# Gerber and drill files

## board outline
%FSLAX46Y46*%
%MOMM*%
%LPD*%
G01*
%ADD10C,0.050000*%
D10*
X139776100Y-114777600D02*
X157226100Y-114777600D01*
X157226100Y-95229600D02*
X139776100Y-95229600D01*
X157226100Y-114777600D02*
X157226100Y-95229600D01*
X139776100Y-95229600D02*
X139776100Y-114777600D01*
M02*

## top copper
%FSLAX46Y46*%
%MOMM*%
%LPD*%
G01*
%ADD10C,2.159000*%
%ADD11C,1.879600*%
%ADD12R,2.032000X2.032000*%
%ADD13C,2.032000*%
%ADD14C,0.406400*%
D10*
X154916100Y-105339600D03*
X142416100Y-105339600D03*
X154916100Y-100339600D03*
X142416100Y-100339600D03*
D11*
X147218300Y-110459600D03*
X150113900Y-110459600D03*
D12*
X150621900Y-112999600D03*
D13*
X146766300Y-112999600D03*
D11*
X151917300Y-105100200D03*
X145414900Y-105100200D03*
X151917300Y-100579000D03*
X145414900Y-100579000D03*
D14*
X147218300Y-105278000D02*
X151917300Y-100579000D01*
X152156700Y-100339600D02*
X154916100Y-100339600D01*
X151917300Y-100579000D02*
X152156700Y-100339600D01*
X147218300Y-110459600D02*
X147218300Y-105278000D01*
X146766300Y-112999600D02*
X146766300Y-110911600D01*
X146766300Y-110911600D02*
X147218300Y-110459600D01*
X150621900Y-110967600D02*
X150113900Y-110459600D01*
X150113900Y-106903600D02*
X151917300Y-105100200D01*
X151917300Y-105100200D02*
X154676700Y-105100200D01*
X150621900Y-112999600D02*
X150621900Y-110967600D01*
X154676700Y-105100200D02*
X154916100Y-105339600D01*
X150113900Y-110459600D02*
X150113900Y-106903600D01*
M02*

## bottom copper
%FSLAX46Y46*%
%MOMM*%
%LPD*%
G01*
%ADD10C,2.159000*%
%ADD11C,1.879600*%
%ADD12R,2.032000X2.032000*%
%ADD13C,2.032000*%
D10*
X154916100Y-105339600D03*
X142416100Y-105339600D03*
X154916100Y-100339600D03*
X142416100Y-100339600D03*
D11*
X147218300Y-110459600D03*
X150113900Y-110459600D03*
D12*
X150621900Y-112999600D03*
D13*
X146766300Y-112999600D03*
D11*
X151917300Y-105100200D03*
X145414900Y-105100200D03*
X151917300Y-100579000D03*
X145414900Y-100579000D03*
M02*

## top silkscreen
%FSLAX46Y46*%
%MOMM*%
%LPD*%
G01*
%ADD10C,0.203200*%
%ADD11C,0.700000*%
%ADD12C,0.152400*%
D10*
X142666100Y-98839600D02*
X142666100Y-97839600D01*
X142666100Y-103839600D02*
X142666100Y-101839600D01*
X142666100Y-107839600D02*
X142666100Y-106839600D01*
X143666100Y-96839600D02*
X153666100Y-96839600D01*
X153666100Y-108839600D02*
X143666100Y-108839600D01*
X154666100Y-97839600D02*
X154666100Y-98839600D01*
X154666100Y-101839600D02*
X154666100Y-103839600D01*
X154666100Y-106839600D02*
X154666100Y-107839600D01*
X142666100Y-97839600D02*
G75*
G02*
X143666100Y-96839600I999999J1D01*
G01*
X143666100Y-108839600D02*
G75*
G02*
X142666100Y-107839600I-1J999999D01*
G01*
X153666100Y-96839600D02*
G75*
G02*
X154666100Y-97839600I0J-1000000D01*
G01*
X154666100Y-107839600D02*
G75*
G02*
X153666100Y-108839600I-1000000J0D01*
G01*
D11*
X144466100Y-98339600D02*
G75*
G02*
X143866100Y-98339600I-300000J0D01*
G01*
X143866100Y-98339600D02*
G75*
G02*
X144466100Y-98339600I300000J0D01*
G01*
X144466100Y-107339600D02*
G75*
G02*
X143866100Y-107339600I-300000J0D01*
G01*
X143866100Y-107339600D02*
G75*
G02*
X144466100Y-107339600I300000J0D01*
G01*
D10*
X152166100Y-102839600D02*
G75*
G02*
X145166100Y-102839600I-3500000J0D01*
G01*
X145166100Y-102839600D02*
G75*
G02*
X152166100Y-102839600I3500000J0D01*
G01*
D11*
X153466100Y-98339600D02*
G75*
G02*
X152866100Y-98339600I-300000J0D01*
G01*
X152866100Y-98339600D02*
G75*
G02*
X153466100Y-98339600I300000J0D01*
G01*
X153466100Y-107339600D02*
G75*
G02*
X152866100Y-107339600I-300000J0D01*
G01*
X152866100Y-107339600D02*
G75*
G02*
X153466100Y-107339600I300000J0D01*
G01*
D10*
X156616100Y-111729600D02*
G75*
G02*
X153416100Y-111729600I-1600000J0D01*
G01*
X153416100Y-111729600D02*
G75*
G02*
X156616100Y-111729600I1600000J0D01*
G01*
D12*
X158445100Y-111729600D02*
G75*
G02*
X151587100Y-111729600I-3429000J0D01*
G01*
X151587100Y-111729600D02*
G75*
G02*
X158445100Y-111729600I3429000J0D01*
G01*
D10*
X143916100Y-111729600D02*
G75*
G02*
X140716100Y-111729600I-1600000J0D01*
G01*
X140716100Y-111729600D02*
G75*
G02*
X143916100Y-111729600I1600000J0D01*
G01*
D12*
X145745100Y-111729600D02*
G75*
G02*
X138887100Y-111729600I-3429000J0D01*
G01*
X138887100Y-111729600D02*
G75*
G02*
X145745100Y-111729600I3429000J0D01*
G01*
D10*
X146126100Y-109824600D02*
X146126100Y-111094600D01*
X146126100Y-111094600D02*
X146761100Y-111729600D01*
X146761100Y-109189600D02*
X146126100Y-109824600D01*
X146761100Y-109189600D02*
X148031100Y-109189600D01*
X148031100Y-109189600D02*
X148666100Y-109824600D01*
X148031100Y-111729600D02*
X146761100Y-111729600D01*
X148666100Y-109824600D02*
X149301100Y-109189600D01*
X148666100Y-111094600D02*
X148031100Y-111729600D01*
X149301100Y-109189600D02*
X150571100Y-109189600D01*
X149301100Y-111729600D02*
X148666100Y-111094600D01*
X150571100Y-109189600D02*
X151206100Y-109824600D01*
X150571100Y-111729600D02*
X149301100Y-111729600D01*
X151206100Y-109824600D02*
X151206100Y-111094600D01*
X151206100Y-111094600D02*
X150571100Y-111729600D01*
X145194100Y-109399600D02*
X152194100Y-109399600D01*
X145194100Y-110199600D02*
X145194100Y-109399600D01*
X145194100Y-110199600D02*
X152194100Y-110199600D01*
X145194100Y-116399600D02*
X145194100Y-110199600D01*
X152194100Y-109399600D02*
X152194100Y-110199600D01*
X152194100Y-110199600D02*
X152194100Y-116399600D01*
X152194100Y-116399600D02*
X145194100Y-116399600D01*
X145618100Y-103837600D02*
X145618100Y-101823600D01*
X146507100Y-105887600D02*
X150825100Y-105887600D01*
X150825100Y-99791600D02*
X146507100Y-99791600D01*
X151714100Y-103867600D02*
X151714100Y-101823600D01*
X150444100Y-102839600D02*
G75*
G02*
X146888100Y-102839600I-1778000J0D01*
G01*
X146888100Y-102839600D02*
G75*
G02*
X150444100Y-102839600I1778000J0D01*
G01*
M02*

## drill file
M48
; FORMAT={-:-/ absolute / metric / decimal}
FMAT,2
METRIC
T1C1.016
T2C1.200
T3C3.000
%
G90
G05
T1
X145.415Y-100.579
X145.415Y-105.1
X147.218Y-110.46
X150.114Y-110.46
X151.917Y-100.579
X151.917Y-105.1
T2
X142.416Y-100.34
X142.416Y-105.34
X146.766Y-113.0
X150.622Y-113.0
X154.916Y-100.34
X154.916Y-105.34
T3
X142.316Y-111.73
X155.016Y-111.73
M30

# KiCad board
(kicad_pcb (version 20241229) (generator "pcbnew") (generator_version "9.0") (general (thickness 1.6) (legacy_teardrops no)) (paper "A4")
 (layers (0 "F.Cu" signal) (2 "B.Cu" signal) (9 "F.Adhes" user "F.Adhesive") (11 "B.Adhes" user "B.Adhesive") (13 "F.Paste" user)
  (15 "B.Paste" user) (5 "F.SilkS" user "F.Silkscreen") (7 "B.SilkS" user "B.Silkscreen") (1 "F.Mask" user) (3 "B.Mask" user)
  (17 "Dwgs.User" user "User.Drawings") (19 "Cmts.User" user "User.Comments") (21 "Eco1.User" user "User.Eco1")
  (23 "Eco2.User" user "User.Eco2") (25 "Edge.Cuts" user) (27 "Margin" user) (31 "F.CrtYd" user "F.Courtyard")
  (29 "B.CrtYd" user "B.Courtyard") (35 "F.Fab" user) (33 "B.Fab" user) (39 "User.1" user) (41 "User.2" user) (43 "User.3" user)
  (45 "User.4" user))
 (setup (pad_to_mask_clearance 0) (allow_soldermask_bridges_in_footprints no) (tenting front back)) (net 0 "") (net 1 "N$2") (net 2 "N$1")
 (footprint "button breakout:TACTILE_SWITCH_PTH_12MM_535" (layer "F.Cu") (at 148.6661 102.8396)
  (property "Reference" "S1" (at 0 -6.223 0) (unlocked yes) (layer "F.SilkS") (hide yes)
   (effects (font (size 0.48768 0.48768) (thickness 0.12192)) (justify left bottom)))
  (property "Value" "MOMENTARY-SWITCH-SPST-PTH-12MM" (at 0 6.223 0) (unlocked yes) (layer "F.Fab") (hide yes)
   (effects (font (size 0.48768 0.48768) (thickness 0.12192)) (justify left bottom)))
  (fp_line (start -6 -4) (end -6 -5) (stroke (width 0.2032) (type solid)) (layer "F.SilkS"))
  (fp_line (start -6 1) (end -6 -1) (stroke (width 0.2032) (type solid)) (layer "F.SilkS"))
  (fp_line (start -6 5) (end -6 4) (stroke (width 0.2032) (type solid)) (layer "F.SilkS"))
  (fp_line (start -5 -6) (end 5 -6) (stroke (width 0.2032) (type solid)) (layer "F.SilkS"))
  (fp_line (start 5 6) (end -5 6) (stroke (width 0.2032) (type solid)) (layer "F.SilkS"))
  (fp_line (start 6 -5) (end 6 -4) (stroke (width 0.2032) (type solid)) (layer "F.SilkS"))
  (fp_line (start 6 -1) (end 6 1) (stroke (width 0.2032) (type solid)) (layer "F.SilkS"))
  (fp_line (start 6 4) (end 6 5) (stroke (width 0.2032) (type solid)) (layer "F.SilkS"))
  (fp_arc (start -6 -5) (mid -5.707107 -5.707107) (end -5 -6) (stroke (width 0.2032) (type solid)) (layer "F.SilkS"))
  (fp_arc (start -5 6) (mid -5.707107 5.707107) (end -6 5) (stroke (width 0.2032) (type solid)) (layer "F.SilkS"))
  (fp_arc (start 5 -6) (mid 5.707107 -5.707107) (end 6 -5) (stroke (width 0.2032) (type solid)) (layer "F.SilkS"))
  (fp_arc (start 6 5) (mid 5.707107 5.707107) (end 5 6) (stroke (width 0.2032) (type solid)) (layer "F.SilkS"))
  (fp_circle (center -4.5 -4.5) (end -4.2 -4.5) (stroke (width 0.7) (type solid)) (fill no) (layer "F.SilkS"))
  (fp_circle (center -4.5 4.5) (end -4.2 4.5) (stroke (width 0.7) (type solid)) (fill no) (layer "F.SilkS"))
  (fp_circle (center 0 0) (end 3.5 0) (stroke (width 0.2032) (type solid)) (fill no) (layer "F.SilkS"))
  (fp_circle (center 4.5 -4.5) (end 4.8 -4.5) (stroke (width 0.7) (type solid)) (fill no) (layer "F.SilkS"))
  (fp_circle (center 4.5 4.5) (end 4.8 4.5) (stroke (width 0.7) (type solid)) (fill no) (layer "F.SilkS"))
  (pad "1" thru_hole circle (at 6.25 2.5) (size 2.159 2.159) (drill 1.2) (layers "*.Cu" "*.Mask") (remove_unused_layers no) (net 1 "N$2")
   (solder_mask_margin 0.0508) (thermal_bridge_angle 0))
  (pad "2" thru_hole circle (at -6.25 2.5) (size 2.159 2.159) (drill 1.2) (layers "*.Cu" "*.Mask") (remove_unused_layers no)
   (solder_mask_margin 0.0508) (thermal_bridge_angle 0))
  (pad "3" thru_hole circle (at 6.25 -2.5) (size 2.159 2.159) (drill 1.2) (layers "*.Cu" "*.Mask") (remove_unused_layers no) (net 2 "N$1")
   (solder_mask_margin 0.0508) (thermal_bridge_angle 0))
  (pad "4" thru_hole circle (at -6.25 -2.5) (size 2.159 2.159) (drill 1.2) (layers "*.Cu" "*.Mask") (remove_unused_layers no)
   (solder_mask_margin 0.0508) (thermal_bridge_angle 0)))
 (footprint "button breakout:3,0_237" (layer "F.Cu") (at 155.0161 111.7296)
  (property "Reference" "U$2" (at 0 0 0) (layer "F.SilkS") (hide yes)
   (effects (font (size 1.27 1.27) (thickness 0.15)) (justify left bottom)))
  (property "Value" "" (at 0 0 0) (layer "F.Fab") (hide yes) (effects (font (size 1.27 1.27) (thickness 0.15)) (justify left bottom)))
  (fp_circle (center 0 0) (end 1.6 0) (stroke (width 0.2032) (type solid)) (fill no) (layer "F.SilkS"))
  (fp_circle (center 0 0) (end 3.429 0) (stroke (width 0.1524) (type solid)) (fill no) (layer "F.SilkS"))
  (pad "" np_thru_hole circle (at 0 0) (size 3 3) (drill 3) (layers "*.Cu" "*.Mask"))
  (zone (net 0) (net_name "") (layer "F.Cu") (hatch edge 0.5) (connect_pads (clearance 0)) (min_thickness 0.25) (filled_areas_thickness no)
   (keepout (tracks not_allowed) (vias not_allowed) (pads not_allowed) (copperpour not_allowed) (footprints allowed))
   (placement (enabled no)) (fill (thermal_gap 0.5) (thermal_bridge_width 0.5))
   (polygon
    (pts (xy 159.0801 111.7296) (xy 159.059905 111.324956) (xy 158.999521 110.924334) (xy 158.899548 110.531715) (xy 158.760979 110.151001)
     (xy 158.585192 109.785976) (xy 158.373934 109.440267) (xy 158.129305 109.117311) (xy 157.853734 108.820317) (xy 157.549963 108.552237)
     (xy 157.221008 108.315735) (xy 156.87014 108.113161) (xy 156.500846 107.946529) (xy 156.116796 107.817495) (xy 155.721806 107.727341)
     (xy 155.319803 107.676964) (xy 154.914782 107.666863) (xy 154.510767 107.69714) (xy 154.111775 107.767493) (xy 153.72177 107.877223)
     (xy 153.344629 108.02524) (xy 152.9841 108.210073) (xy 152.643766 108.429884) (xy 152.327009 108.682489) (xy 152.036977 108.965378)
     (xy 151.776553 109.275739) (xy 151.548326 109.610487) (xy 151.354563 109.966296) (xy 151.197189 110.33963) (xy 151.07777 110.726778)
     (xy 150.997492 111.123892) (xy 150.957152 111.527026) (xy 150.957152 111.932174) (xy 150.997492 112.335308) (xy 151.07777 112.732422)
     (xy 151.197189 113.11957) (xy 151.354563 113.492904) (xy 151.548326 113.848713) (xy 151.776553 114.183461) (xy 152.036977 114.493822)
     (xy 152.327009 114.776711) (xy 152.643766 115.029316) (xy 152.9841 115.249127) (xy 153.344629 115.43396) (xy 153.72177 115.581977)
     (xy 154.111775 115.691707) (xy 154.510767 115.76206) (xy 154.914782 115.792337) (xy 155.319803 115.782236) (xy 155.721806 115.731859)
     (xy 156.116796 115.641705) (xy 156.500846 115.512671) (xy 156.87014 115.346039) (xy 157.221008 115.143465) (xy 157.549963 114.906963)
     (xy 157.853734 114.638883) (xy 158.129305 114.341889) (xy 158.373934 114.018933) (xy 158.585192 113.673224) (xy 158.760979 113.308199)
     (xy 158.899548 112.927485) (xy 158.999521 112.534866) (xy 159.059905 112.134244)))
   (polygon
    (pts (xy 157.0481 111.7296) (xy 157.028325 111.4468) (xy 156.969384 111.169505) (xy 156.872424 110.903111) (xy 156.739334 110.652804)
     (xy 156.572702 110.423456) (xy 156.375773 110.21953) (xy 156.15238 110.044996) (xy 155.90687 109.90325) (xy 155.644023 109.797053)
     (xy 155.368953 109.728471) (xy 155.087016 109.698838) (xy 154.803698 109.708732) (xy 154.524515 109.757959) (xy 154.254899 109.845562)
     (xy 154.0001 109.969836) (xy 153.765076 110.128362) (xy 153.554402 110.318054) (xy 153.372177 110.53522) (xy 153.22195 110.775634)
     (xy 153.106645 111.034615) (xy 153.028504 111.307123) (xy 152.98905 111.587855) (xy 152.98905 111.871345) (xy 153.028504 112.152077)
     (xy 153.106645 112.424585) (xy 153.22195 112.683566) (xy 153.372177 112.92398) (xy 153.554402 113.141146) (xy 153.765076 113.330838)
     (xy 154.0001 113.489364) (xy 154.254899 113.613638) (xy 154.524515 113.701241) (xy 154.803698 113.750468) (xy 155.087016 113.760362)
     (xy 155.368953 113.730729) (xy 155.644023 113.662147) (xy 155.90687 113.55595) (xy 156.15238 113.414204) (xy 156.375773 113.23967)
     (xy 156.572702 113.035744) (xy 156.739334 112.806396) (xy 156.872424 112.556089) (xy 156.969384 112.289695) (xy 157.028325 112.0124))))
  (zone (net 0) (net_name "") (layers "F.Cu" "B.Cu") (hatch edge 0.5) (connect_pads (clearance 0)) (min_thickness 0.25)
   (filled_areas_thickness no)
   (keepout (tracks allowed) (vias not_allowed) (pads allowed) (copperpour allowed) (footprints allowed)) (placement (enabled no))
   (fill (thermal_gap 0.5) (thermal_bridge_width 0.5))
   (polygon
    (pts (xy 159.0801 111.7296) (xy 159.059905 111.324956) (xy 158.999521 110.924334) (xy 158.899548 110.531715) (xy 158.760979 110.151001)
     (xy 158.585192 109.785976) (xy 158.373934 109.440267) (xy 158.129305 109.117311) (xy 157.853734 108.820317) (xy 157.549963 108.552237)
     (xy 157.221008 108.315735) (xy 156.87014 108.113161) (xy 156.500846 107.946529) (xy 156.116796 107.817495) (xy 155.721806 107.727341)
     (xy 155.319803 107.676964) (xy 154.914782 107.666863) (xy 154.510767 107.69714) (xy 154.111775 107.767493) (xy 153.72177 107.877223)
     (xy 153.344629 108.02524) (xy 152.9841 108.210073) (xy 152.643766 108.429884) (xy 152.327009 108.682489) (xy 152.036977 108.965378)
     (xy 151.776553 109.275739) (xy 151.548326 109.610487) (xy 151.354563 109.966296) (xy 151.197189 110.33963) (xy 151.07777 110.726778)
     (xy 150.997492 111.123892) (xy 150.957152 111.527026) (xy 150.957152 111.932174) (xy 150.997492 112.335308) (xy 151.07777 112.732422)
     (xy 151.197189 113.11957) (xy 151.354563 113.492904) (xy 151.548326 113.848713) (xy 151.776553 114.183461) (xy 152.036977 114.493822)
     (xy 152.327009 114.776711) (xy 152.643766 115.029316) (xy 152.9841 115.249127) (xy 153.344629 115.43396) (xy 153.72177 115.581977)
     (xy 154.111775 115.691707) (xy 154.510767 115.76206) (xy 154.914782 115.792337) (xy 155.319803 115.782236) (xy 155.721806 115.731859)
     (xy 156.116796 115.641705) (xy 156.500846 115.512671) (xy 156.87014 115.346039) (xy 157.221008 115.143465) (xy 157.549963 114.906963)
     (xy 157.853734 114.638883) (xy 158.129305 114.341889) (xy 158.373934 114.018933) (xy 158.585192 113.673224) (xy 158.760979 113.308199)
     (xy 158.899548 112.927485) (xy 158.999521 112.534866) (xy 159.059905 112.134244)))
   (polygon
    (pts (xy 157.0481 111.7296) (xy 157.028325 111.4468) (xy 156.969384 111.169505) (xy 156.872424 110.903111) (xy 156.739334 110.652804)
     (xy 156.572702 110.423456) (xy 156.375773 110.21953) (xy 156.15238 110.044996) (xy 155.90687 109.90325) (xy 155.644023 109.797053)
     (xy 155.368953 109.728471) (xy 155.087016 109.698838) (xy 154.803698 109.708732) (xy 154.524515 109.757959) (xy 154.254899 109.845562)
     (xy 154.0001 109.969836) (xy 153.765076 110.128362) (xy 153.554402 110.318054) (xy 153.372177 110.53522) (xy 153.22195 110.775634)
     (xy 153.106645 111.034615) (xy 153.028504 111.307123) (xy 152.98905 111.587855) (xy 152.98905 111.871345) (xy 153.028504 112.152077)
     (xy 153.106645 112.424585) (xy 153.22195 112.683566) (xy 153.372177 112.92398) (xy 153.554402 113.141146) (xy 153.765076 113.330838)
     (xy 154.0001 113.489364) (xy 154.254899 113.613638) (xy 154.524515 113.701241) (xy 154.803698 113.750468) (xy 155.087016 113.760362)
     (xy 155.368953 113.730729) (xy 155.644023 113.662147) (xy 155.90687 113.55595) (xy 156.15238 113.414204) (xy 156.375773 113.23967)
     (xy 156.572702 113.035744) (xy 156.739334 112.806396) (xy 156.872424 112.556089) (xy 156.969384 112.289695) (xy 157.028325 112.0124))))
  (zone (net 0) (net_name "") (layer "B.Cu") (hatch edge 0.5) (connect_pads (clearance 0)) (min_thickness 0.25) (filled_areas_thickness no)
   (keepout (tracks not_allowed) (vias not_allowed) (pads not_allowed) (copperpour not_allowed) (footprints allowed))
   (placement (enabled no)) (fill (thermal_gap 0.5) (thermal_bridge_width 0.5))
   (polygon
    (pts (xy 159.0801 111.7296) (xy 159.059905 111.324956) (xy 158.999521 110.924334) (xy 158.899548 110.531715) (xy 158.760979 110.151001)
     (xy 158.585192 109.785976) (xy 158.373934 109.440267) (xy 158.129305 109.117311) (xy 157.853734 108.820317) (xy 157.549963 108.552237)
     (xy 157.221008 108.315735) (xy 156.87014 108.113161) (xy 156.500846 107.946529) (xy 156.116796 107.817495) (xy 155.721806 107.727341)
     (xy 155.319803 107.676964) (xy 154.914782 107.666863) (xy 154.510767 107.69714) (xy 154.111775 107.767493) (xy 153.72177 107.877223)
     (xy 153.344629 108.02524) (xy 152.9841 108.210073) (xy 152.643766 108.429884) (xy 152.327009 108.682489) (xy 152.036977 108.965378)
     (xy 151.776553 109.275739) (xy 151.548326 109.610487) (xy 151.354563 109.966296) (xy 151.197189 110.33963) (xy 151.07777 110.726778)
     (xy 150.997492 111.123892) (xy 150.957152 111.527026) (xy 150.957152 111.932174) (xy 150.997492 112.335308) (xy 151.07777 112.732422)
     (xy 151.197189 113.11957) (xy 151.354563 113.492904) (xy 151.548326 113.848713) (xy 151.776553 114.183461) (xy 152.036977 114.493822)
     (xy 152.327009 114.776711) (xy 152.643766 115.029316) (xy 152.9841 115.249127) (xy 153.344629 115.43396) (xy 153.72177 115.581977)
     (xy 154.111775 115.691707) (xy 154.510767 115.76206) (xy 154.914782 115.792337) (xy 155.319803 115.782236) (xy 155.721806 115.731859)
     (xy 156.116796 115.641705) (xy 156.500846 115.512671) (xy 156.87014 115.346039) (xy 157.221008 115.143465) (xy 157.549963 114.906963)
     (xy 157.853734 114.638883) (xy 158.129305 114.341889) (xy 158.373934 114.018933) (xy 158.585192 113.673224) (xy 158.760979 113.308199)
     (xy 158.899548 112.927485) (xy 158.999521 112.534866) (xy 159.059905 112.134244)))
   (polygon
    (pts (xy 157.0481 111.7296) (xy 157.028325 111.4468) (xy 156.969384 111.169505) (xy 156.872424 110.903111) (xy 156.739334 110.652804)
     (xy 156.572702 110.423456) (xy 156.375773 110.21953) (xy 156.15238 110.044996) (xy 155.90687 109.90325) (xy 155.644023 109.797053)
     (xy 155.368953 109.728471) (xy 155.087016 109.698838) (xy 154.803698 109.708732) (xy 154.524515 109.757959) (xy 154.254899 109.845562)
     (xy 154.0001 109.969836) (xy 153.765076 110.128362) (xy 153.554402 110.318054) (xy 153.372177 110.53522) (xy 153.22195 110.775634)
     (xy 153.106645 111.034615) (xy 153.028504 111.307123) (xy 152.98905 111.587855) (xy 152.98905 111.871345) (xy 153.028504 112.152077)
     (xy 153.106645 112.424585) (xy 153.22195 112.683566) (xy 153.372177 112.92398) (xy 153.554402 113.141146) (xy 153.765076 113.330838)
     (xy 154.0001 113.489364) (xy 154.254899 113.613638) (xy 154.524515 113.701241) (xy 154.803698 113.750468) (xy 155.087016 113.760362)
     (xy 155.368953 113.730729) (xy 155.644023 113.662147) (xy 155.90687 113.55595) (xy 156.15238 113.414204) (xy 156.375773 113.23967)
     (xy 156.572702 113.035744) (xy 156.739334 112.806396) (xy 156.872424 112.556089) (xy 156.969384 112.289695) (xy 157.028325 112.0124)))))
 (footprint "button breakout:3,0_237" (layer "F.Cu") (at 142.3161 111.7296)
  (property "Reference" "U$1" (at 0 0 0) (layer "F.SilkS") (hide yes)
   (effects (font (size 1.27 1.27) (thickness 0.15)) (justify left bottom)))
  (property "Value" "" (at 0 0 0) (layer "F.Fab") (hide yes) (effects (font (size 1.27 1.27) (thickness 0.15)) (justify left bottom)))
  (fp_circle (center 0 0) (end 1.6 0) (stroke (width 0.2032) (type solid)) (fill no) (layer "F.SilkS"))
  (fp_circle (center 0 0) (end 3.429 0) (stroke (width 0.1524) (type solid)) (fill no) (layer "F.SilkS"))
  (pad "" np_thru_hole circle (at 0 0) (size 3 3) (drill 3) (layers "*.Cu" "*.Mask"))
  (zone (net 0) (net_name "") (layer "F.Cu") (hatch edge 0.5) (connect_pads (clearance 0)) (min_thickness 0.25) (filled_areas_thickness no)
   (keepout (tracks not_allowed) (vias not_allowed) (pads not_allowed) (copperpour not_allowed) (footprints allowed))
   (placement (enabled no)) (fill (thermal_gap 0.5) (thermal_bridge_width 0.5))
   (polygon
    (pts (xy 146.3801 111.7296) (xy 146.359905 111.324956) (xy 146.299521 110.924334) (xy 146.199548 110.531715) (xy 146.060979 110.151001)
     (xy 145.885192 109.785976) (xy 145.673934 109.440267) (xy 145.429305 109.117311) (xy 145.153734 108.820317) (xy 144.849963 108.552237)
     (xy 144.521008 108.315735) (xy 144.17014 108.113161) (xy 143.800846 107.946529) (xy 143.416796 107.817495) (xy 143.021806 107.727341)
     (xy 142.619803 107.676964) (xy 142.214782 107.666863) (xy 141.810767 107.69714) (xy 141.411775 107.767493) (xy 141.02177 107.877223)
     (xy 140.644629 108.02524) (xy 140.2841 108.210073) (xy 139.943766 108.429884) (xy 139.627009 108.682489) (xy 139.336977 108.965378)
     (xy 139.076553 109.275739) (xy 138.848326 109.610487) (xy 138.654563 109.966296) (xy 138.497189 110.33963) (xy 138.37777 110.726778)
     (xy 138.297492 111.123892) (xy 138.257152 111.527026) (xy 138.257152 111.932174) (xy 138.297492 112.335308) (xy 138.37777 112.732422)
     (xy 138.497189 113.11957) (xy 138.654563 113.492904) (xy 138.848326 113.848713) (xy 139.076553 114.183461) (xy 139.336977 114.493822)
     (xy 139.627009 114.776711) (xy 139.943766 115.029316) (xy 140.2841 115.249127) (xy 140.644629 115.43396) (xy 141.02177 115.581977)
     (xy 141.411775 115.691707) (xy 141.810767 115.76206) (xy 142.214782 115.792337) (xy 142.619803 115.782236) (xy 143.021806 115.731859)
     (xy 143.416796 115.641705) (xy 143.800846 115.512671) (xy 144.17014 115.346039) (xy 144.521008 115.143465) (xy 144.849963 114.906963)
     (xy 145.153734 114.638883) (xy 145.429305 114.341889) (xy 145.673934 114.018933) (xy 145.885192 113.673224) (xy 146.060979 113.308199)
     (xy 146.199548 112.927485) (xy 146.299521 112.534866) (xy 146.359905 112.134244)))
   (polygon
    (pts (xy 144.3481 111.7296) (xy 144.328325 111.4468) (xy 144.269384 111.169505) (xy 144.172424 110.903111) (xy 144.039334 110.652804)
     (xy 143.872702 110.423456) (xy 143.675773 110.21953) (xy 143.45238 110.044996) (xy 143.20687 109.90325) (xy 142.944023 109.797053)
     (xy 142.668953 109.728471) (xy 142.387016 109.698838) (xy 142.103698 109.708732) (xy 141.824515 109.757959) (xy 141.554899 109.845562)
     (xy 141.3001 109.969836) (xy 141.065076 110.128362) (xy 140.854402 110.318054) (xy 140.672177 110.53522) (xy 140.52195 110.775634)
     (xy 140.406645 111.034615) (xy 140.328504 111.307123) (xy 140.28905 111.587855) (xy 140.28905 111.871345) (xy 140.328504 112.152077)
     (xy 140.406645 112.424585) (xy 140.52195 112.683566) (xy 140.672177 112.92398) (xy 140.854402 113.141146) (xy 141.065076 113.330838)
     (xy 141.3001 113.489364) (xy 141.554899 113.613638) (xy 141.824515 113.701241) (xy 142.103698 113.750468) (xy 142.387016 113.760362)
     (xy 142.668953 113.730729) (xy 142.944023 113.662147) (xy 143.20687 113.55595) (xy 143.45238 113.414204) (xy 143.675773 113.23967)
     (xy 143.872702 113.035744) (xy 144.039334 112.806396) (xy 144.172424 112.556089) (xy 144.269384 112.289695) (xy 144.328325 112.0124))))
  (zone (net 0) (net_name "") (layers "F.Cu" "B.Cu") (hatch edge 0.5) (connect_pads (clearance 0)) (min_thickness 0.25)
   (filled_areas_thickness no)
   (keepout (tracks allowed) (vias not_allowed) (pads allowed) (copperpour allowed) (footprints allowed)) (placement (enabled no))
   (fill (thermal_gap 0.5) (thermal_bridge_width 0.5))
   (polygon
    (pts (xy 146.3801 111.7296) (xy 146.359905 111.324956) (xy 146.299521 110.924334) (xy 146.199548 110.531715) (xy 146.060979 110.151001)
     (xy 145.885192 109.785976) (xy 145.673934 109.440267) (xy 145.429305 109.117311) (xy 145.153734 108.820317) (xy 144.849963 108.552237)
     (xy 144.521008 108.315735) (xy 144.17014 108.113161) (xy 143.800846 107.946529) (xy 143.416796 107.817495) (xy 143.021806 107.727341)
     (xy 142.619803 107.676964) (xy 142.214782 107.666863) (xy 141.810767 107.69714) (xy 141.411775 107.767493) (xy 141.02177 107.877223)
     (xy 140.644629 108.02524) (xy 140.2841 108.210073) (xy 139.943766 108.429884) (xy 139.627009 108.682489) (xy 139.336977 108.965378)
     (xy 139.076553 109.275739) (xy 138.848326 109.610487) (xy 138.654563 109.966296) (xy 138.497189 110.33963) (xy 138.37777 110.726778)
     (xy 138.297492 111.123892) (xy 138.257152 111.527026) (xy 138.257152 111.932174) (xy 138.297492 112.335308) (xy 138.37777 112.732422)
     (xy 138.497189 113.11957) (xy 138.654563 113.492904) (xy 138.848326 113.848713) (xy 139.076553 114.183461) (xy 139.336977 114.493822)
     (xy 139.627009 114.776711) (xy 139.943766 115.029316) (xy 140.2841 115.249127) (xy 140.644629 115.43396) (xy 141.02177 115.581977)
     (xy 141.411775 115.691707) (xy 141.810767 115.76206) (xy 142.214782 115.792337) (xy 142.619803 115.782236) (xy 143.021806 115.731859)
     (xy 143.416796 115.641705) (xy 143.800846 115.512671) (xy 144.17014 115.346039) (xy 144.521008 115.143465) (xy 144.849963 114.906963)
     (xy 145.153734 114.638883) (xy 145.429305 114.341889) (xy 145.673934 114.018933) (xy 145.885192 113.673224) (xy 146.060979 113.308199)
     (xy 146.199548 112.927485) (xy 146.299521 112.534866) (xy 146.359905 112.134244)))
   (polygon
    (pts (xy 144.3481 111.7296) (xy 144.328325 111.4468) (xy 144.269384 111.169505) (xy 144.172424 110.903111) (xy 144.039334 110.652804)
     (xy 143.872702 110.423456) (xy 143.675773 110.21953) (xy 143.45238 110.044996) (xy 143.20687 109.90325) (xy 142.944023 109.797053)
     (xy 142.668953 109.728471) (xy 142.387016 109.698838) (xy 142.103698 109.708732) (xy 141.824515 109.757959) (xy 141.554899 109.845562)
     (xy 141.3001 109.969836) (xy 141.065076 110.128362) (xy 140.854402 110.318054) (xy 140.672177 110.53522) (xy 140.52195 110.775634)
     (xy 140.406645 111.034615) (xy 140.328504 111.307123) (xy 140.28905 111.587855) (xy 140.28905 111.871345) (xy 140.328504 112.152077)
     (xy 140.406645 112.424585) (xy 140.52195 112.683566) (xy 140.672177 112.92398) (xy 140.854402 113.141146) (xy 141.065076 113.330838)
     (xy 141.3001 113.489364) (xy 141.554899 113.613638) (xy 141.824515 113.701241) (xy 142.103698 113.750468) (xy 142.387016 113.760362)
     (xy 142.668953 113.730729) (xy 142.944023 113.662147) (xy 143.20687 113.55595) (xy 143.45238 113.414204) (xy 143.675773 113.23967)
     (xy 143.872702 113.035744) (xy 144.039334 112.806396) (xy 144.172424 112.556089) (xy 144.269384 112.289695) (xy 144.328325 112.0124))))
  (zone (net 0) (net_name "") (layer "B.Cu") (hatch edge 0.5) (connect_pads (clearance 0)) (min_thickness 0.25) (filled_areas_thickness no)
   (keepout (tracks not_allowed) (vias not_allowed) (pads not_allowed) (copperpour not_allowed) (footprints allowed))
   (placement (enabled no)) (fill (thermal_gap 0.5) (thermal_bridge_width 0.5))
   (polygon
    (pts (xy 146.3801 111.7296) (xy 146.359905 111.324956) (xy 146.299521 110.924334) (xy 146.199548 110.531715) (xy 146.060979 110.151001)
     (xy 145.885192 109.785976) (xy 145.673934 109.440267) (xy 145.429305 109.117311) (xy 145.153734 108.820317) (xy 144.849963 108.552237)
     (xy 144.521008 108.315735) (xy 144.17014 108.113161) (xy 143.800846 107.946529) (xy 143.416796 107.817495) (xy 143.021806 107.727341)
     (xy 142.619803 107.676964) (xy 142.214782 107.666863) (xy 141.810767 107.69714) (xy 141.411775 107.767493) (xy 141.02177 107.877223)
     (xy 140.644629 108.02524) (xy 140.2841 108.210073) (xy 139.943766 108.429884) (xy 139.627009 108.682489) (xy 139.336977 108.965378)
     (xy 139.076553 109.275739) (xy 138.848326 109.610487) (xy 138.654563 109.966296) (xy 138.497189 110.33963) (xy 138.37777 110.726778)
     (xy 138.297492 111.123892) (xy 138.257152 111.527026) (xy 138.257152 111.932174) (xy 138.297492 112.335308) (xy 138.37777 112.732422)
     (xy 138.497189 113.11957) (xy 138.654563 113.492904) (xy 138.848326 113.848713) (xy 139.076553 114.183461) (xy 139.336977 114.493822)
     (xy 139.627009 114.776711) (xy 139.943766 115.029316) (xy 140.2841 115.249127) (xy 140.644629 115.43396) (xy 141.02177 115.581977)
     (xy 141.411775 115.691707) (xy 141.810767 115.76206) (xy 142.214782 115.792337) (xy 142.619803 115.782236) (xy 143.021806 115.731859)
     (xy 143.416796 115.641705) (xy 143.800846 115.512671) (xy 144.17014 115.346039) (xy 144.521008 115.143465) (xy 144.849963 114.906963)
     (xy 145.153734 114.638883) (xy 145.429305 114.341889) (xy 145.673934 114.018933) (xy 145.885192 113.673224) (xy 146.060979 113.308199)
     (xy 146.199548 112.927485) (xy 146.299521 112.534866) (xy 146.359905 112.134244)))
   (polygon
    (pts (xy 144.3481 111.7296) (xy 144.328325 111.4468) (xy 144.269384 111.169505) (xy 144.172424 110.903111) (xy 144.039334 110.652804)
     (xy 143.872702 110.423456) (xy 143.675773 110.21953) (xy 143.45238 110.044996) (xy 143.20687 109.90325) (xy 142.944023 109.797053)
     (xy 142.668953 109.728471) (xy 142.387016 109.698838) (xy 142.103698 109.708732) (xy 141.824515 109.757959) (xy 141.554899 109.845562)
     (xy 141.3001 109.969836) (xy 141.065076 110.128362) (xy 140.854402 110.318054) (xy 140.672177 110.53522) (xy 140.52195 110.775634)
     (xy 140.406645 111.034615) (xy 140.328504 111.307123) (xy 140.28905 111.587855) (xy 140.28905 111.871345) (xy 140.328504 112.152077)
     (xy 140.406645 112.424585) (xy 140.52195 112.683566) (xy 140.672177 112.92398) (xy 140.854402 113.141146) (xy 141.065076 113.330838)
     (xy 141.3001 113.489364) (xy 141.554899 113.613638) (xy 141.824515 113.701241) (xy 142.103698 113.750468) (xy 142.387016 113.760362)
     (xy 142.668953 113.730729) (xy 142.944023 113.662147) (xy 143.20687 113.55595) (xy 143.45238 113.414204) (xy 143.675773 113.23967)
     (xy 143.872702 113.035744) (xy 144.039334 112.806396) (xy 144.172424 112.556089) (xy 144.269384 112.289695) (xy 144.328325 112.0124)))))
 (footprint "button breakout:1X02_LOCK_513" (layer "F.Cu") (at 147.3961 110.4596)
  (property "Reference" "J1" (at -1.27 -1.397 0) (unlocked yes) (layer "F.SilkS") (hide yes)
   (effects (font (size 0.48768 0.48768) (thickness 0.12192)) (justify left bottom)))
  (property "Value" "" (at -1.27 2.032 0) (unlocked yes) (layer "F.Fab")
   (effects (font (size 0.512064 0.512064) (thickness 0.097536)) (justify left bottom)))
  (fp_line (start -1.27 -0.635) (end -1.27 0.635) (stroke (width 0.2032) (type solid)) (layer "F.SilkS"))
  (fp_line (start -1.27 0.635) (end -0.635 1.27) (stroke (width 0.2032) (type solid)) (layer "F.SilkS"))
  (fp_line (start -0.635 -1.27) (end -1.27 -0.635) (stroke (width 0.2032) (type solid)) (layer "F.SilkS"))
  (fp_line (start -0.635 -1.27) (end 0.635 -1.27) (stroke (width 0.2032) (type solid)) (layer "F.SilkS"))
  (fp_line (start 0.635 -1.27) (end 1.27 -0.635) (stroke (width 0.2032) (type solid)) (layer "F.SilkS"))
  (fp_line (start 0.635 1.27) (end -0.635 1.27) (stroke (width 0.2032) (type solid)) (layer "F.SilkS"))
  (fp_line (start 1.27 -0.635) (end 1.905 -1.27) (stroke (width 0.2032) (type solid)) (layer "F.SilkS"))
  (fp_line (start 1.27 0.635) (end 0.635 1.27) (stroke (width 0.2032) (type solid)) (layer "F.SilkS"))
  (fp_line (start 1.905 -1.27) (end 3.175 -1.27) (stroke (width 0.2032) (type solid)) (layer "F.SilkS"))
  (fp_line (start 1.905 1.27) (end 1.27 0.635) (stroke (width 0.2032) (type solid)) (layer "F.SilkS"))
  (fp_line (start 3.175 -1.27) (end 3.81 -0.635) (stroke (width 0.2032) (type solid)) (layer "F.SilkS"))
  (fp_line (start 3.175 1.27) (end 1.905 1.27) (stroke (width 0.2032) (type solid)) (layer "F.SilkS"))
  (fp_line (start 3.81 -0.635) (end 3.81 0.635) (stroke (width 0.2032) (type solid)) (layer "F.SilkS"))
  (fp_line (start 3.81 0.635) (end 3.175 1.27) (stroke (width 0.2032) (type solid)) (layer "F.SilkS"))
  (pad "1" thru_hole circle (at -0.1778 0 90) (size 1.8796 1.8796) (drill 1.016) (layers "*.Cu" "*.Mask") (remove_unused_layers no)
   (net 2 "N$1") (solder_mask_margin 0.0508) (thermal_bridge_angle 0))
  (pad "2" thru_hole circle (at 2.7178 0 90) (size 1.8796 1.8796) (drill 1.016) (layers "*.Cu" "*.Mask") (remove_unused_layers no)
   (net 1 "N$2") (solder_mask_margin 0.0508) (thermal_bridge_angle 0)))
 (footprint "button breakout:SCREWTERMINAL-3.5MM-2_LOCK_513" (layer "F.Cu") (at 150.4441 112.9996 180)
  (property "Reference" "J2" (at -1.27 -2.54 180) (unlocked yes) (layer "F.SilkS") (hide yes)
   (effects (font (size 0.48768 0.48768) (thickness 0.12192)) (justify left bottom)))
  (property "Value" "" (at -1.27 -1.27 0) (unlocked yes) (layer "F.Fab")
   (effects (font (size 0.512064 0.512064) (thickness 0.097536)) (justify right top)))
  (fp_line (start 5.25 3.6) (end -1.75 3.6) (stroke (width 0.2032) (type solid)) (layer "F.SilkS"))
  (fp_line (start 5.25 2.8) (end 5.25 3.6) (stroke (width 0.2032) (type solid)) (layer "F.SilkS"))
  (fp_line (start 5.25 2.8) (end -1.75 2.8) (stroke (width 0.2032) (type solid)) (layer "F.SilkS"))
  (fp_line (start 5.25 -3.4) (end 5.25 2.8) (stroke (width 0.2032) (type solid)) (layer "F.SilkS"))
  (fp_line (start -1.75 3.6) (end -1.75 2.8) (stroke (width 0.2032) (type solid)) (layer "F.SilkS"))
  (fp_line (start -1.75 2.8) (end -1.75 -3.4) (stroke (width 0.2032) (type solid)) (layer "F.SilkS"))
  (fp_line (start -1.75 -3.4) (end 5.25 -3.4) (stroke (width 0.2032) (type solid)) (layer "F.SilkS"))
  (pad "1" thru_hole rect (at -0.1778 0 180) (size 2.032 2.032) (drill 1.2) (layers "*.Cu" "*.Mask") (remove_unused_layers no) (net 1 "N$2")
   (solder_mask_margin 0.0508) (thermal_bridge_angle 0))
  (pad "2" thru_hole circle (at 3.6778 0 180) (size 2.032 2.032) (drill 1.2) (layers "*.Cu" "*.Mask") (remove_unused_layers no)
   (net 2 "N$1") (solder_mask_margin 0.0508) (thermal_bridge_angle 0)))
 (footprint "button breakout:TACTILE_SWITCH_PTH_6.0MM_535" (layer "F.Cu") (at 148.6661 102.8396 180)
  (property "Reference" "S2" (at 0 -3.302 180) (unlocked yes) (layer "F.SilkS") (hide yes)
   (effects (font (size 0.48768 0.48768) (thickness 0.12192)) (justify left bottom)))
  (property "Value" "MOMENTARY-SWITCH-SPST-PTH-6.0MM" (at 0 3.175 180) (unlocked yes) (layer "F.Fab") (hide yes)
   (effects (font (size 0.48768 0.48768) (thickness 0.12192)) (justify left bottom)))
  (fp_line (start 3.048 -0.998) (end 3.048 1.016) (stroke (width 0.2032) (type solid)) (layer "F.SilkS"))
  (fp_line (start 2.159 -3.048) (end -2.159 -3.048) (stroke (width 0.2032) (type solid)) (layer "F.SilkS"))
  (fp_line (start -2.159 3.048) (end 2.159 3.048) (stroke (width 0.2032) (type solid)) (layer "F.SilkS"))
  (fp_line (start -3.048 -1.028) (end -3.048 1.016) (stroke (width 0.2032) (type solid)) (layer "F.SilkS"))
  (fp_circle (center 0 0) (end 1.778 0) (stroke (width 0.2032) (type solid)) (fill no) (layer "F.SilkS"))
  (pad "1" thru_hole circle (at -3.2512 -2.2606 180) (size 1.8796 1.8796) (drill 1.016) (layers "*.Cu" "*.Mask") (remove_unused_layers no)
   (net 1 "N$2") (solder_mask_margin 0.0508) (thermal_bridge_angle 0))
  (pad "2" thru_hole circle (at 3.2512 -2.2606 180) (size 1.8796 1.8796) (drill 1.016) (layers "*.Cu" "*.Mask") (remove_unused_layers no)
   (solder_mask_margin 0.0508) (thermal_bridge_angle 0))
  (pad "3" thru_hole circle (at -3.2512 2.2606 180) (size 1.8796 1.8796) (drill 1.016) (layers "*.Cu" "*.Mask") (remove_unused_layers no)
   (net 2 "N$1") (solder_mask_margin 0.0508) (thermal_bridge_angle 0))
  (pad "4" thru_hole circle (at 3.2512 2.2606 180) (size 1.8796 1.8796) (drill 1.016) (layers "*.Cu" "*.Mask") (remove_unused_layers no)
   (solder_mask_margin 0.0508) (thermal_bridge_angle 0)))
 (gr_line (start 139.7761 114.7776) (end 157.2261 114.7776) (stroke (width 0.05) (type solid)) (layer "Edge.Cuts"))
 (gr_line (start 157.2261 95.2296) (end 139.7761 95.2296) (stroke (width 0.05) (type solid)) (layer "Edge.Cuts"))
 (gr_line (start 157.2261 114.7776) (end 157.2261 95.2296) (stroke (width 0.05) (type solid)) (layer "Edge.Cuts"))
 (gr_line (start 139.7761 95.2296) (end 139.7761 114.7776) (stroke (width 0.05) (type solid)) (layer "Edge.Cuts"))
 (segment (start 147.2183 105.278) (end 151.9173 100.579) (width 0.4064) (layer "F.Cu") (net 2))
 (segment (start 152.1567 100.3396) (end 154.9161 100.3396) (width 0.4064) (layer "F.Cu") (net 2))
 (segment (start 151.9173 100.579) (end 152.1567 100.3396) (width 0.4064) (layer "F.Cu") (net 2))
 (segment (start 147.2183 110.4596) (end 147.2183 105.278) (width 0.4064) (layer "F.Cu") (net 2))
 (segment (start 146.7663 112.9996) (end 146.7663 110.9116) (width 0.4064) (layer "F.Cu") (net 2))
 (segment (start 146.7663 110.9116) (end 147.2183 110.4596) (width 0.4064) (layer "F.Cu") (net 2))
 (segment (start 150.6219 110.9676) (end 150.1139 110.4596) (width 0.4064) (layer "F.Cu") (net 1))
 (segment (start 150.1139 106.9036) (end 151.9173 105.1002) (width 0.4064) (layer "F.Cu") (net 1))
 (segment (start 151.9173 105.1002) (end 154.6767 105.1002) (width 0.4064) (layer "F.Cu") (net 1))
 (segment (start 150.6219 112.9996) (end 150.6219 110.9676) (width 0.4064) (layer "F.Cu") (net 1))
 (segment (start 154.6767 105.1002) (end 154.9161 105.3396) (width 0.4064) (layer "F.Cu") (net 1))
 (segment (start 150.1139 110.4596) (end 150.1139 106.9036) (width 0.4064) (layer "F.Cu") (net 1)))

